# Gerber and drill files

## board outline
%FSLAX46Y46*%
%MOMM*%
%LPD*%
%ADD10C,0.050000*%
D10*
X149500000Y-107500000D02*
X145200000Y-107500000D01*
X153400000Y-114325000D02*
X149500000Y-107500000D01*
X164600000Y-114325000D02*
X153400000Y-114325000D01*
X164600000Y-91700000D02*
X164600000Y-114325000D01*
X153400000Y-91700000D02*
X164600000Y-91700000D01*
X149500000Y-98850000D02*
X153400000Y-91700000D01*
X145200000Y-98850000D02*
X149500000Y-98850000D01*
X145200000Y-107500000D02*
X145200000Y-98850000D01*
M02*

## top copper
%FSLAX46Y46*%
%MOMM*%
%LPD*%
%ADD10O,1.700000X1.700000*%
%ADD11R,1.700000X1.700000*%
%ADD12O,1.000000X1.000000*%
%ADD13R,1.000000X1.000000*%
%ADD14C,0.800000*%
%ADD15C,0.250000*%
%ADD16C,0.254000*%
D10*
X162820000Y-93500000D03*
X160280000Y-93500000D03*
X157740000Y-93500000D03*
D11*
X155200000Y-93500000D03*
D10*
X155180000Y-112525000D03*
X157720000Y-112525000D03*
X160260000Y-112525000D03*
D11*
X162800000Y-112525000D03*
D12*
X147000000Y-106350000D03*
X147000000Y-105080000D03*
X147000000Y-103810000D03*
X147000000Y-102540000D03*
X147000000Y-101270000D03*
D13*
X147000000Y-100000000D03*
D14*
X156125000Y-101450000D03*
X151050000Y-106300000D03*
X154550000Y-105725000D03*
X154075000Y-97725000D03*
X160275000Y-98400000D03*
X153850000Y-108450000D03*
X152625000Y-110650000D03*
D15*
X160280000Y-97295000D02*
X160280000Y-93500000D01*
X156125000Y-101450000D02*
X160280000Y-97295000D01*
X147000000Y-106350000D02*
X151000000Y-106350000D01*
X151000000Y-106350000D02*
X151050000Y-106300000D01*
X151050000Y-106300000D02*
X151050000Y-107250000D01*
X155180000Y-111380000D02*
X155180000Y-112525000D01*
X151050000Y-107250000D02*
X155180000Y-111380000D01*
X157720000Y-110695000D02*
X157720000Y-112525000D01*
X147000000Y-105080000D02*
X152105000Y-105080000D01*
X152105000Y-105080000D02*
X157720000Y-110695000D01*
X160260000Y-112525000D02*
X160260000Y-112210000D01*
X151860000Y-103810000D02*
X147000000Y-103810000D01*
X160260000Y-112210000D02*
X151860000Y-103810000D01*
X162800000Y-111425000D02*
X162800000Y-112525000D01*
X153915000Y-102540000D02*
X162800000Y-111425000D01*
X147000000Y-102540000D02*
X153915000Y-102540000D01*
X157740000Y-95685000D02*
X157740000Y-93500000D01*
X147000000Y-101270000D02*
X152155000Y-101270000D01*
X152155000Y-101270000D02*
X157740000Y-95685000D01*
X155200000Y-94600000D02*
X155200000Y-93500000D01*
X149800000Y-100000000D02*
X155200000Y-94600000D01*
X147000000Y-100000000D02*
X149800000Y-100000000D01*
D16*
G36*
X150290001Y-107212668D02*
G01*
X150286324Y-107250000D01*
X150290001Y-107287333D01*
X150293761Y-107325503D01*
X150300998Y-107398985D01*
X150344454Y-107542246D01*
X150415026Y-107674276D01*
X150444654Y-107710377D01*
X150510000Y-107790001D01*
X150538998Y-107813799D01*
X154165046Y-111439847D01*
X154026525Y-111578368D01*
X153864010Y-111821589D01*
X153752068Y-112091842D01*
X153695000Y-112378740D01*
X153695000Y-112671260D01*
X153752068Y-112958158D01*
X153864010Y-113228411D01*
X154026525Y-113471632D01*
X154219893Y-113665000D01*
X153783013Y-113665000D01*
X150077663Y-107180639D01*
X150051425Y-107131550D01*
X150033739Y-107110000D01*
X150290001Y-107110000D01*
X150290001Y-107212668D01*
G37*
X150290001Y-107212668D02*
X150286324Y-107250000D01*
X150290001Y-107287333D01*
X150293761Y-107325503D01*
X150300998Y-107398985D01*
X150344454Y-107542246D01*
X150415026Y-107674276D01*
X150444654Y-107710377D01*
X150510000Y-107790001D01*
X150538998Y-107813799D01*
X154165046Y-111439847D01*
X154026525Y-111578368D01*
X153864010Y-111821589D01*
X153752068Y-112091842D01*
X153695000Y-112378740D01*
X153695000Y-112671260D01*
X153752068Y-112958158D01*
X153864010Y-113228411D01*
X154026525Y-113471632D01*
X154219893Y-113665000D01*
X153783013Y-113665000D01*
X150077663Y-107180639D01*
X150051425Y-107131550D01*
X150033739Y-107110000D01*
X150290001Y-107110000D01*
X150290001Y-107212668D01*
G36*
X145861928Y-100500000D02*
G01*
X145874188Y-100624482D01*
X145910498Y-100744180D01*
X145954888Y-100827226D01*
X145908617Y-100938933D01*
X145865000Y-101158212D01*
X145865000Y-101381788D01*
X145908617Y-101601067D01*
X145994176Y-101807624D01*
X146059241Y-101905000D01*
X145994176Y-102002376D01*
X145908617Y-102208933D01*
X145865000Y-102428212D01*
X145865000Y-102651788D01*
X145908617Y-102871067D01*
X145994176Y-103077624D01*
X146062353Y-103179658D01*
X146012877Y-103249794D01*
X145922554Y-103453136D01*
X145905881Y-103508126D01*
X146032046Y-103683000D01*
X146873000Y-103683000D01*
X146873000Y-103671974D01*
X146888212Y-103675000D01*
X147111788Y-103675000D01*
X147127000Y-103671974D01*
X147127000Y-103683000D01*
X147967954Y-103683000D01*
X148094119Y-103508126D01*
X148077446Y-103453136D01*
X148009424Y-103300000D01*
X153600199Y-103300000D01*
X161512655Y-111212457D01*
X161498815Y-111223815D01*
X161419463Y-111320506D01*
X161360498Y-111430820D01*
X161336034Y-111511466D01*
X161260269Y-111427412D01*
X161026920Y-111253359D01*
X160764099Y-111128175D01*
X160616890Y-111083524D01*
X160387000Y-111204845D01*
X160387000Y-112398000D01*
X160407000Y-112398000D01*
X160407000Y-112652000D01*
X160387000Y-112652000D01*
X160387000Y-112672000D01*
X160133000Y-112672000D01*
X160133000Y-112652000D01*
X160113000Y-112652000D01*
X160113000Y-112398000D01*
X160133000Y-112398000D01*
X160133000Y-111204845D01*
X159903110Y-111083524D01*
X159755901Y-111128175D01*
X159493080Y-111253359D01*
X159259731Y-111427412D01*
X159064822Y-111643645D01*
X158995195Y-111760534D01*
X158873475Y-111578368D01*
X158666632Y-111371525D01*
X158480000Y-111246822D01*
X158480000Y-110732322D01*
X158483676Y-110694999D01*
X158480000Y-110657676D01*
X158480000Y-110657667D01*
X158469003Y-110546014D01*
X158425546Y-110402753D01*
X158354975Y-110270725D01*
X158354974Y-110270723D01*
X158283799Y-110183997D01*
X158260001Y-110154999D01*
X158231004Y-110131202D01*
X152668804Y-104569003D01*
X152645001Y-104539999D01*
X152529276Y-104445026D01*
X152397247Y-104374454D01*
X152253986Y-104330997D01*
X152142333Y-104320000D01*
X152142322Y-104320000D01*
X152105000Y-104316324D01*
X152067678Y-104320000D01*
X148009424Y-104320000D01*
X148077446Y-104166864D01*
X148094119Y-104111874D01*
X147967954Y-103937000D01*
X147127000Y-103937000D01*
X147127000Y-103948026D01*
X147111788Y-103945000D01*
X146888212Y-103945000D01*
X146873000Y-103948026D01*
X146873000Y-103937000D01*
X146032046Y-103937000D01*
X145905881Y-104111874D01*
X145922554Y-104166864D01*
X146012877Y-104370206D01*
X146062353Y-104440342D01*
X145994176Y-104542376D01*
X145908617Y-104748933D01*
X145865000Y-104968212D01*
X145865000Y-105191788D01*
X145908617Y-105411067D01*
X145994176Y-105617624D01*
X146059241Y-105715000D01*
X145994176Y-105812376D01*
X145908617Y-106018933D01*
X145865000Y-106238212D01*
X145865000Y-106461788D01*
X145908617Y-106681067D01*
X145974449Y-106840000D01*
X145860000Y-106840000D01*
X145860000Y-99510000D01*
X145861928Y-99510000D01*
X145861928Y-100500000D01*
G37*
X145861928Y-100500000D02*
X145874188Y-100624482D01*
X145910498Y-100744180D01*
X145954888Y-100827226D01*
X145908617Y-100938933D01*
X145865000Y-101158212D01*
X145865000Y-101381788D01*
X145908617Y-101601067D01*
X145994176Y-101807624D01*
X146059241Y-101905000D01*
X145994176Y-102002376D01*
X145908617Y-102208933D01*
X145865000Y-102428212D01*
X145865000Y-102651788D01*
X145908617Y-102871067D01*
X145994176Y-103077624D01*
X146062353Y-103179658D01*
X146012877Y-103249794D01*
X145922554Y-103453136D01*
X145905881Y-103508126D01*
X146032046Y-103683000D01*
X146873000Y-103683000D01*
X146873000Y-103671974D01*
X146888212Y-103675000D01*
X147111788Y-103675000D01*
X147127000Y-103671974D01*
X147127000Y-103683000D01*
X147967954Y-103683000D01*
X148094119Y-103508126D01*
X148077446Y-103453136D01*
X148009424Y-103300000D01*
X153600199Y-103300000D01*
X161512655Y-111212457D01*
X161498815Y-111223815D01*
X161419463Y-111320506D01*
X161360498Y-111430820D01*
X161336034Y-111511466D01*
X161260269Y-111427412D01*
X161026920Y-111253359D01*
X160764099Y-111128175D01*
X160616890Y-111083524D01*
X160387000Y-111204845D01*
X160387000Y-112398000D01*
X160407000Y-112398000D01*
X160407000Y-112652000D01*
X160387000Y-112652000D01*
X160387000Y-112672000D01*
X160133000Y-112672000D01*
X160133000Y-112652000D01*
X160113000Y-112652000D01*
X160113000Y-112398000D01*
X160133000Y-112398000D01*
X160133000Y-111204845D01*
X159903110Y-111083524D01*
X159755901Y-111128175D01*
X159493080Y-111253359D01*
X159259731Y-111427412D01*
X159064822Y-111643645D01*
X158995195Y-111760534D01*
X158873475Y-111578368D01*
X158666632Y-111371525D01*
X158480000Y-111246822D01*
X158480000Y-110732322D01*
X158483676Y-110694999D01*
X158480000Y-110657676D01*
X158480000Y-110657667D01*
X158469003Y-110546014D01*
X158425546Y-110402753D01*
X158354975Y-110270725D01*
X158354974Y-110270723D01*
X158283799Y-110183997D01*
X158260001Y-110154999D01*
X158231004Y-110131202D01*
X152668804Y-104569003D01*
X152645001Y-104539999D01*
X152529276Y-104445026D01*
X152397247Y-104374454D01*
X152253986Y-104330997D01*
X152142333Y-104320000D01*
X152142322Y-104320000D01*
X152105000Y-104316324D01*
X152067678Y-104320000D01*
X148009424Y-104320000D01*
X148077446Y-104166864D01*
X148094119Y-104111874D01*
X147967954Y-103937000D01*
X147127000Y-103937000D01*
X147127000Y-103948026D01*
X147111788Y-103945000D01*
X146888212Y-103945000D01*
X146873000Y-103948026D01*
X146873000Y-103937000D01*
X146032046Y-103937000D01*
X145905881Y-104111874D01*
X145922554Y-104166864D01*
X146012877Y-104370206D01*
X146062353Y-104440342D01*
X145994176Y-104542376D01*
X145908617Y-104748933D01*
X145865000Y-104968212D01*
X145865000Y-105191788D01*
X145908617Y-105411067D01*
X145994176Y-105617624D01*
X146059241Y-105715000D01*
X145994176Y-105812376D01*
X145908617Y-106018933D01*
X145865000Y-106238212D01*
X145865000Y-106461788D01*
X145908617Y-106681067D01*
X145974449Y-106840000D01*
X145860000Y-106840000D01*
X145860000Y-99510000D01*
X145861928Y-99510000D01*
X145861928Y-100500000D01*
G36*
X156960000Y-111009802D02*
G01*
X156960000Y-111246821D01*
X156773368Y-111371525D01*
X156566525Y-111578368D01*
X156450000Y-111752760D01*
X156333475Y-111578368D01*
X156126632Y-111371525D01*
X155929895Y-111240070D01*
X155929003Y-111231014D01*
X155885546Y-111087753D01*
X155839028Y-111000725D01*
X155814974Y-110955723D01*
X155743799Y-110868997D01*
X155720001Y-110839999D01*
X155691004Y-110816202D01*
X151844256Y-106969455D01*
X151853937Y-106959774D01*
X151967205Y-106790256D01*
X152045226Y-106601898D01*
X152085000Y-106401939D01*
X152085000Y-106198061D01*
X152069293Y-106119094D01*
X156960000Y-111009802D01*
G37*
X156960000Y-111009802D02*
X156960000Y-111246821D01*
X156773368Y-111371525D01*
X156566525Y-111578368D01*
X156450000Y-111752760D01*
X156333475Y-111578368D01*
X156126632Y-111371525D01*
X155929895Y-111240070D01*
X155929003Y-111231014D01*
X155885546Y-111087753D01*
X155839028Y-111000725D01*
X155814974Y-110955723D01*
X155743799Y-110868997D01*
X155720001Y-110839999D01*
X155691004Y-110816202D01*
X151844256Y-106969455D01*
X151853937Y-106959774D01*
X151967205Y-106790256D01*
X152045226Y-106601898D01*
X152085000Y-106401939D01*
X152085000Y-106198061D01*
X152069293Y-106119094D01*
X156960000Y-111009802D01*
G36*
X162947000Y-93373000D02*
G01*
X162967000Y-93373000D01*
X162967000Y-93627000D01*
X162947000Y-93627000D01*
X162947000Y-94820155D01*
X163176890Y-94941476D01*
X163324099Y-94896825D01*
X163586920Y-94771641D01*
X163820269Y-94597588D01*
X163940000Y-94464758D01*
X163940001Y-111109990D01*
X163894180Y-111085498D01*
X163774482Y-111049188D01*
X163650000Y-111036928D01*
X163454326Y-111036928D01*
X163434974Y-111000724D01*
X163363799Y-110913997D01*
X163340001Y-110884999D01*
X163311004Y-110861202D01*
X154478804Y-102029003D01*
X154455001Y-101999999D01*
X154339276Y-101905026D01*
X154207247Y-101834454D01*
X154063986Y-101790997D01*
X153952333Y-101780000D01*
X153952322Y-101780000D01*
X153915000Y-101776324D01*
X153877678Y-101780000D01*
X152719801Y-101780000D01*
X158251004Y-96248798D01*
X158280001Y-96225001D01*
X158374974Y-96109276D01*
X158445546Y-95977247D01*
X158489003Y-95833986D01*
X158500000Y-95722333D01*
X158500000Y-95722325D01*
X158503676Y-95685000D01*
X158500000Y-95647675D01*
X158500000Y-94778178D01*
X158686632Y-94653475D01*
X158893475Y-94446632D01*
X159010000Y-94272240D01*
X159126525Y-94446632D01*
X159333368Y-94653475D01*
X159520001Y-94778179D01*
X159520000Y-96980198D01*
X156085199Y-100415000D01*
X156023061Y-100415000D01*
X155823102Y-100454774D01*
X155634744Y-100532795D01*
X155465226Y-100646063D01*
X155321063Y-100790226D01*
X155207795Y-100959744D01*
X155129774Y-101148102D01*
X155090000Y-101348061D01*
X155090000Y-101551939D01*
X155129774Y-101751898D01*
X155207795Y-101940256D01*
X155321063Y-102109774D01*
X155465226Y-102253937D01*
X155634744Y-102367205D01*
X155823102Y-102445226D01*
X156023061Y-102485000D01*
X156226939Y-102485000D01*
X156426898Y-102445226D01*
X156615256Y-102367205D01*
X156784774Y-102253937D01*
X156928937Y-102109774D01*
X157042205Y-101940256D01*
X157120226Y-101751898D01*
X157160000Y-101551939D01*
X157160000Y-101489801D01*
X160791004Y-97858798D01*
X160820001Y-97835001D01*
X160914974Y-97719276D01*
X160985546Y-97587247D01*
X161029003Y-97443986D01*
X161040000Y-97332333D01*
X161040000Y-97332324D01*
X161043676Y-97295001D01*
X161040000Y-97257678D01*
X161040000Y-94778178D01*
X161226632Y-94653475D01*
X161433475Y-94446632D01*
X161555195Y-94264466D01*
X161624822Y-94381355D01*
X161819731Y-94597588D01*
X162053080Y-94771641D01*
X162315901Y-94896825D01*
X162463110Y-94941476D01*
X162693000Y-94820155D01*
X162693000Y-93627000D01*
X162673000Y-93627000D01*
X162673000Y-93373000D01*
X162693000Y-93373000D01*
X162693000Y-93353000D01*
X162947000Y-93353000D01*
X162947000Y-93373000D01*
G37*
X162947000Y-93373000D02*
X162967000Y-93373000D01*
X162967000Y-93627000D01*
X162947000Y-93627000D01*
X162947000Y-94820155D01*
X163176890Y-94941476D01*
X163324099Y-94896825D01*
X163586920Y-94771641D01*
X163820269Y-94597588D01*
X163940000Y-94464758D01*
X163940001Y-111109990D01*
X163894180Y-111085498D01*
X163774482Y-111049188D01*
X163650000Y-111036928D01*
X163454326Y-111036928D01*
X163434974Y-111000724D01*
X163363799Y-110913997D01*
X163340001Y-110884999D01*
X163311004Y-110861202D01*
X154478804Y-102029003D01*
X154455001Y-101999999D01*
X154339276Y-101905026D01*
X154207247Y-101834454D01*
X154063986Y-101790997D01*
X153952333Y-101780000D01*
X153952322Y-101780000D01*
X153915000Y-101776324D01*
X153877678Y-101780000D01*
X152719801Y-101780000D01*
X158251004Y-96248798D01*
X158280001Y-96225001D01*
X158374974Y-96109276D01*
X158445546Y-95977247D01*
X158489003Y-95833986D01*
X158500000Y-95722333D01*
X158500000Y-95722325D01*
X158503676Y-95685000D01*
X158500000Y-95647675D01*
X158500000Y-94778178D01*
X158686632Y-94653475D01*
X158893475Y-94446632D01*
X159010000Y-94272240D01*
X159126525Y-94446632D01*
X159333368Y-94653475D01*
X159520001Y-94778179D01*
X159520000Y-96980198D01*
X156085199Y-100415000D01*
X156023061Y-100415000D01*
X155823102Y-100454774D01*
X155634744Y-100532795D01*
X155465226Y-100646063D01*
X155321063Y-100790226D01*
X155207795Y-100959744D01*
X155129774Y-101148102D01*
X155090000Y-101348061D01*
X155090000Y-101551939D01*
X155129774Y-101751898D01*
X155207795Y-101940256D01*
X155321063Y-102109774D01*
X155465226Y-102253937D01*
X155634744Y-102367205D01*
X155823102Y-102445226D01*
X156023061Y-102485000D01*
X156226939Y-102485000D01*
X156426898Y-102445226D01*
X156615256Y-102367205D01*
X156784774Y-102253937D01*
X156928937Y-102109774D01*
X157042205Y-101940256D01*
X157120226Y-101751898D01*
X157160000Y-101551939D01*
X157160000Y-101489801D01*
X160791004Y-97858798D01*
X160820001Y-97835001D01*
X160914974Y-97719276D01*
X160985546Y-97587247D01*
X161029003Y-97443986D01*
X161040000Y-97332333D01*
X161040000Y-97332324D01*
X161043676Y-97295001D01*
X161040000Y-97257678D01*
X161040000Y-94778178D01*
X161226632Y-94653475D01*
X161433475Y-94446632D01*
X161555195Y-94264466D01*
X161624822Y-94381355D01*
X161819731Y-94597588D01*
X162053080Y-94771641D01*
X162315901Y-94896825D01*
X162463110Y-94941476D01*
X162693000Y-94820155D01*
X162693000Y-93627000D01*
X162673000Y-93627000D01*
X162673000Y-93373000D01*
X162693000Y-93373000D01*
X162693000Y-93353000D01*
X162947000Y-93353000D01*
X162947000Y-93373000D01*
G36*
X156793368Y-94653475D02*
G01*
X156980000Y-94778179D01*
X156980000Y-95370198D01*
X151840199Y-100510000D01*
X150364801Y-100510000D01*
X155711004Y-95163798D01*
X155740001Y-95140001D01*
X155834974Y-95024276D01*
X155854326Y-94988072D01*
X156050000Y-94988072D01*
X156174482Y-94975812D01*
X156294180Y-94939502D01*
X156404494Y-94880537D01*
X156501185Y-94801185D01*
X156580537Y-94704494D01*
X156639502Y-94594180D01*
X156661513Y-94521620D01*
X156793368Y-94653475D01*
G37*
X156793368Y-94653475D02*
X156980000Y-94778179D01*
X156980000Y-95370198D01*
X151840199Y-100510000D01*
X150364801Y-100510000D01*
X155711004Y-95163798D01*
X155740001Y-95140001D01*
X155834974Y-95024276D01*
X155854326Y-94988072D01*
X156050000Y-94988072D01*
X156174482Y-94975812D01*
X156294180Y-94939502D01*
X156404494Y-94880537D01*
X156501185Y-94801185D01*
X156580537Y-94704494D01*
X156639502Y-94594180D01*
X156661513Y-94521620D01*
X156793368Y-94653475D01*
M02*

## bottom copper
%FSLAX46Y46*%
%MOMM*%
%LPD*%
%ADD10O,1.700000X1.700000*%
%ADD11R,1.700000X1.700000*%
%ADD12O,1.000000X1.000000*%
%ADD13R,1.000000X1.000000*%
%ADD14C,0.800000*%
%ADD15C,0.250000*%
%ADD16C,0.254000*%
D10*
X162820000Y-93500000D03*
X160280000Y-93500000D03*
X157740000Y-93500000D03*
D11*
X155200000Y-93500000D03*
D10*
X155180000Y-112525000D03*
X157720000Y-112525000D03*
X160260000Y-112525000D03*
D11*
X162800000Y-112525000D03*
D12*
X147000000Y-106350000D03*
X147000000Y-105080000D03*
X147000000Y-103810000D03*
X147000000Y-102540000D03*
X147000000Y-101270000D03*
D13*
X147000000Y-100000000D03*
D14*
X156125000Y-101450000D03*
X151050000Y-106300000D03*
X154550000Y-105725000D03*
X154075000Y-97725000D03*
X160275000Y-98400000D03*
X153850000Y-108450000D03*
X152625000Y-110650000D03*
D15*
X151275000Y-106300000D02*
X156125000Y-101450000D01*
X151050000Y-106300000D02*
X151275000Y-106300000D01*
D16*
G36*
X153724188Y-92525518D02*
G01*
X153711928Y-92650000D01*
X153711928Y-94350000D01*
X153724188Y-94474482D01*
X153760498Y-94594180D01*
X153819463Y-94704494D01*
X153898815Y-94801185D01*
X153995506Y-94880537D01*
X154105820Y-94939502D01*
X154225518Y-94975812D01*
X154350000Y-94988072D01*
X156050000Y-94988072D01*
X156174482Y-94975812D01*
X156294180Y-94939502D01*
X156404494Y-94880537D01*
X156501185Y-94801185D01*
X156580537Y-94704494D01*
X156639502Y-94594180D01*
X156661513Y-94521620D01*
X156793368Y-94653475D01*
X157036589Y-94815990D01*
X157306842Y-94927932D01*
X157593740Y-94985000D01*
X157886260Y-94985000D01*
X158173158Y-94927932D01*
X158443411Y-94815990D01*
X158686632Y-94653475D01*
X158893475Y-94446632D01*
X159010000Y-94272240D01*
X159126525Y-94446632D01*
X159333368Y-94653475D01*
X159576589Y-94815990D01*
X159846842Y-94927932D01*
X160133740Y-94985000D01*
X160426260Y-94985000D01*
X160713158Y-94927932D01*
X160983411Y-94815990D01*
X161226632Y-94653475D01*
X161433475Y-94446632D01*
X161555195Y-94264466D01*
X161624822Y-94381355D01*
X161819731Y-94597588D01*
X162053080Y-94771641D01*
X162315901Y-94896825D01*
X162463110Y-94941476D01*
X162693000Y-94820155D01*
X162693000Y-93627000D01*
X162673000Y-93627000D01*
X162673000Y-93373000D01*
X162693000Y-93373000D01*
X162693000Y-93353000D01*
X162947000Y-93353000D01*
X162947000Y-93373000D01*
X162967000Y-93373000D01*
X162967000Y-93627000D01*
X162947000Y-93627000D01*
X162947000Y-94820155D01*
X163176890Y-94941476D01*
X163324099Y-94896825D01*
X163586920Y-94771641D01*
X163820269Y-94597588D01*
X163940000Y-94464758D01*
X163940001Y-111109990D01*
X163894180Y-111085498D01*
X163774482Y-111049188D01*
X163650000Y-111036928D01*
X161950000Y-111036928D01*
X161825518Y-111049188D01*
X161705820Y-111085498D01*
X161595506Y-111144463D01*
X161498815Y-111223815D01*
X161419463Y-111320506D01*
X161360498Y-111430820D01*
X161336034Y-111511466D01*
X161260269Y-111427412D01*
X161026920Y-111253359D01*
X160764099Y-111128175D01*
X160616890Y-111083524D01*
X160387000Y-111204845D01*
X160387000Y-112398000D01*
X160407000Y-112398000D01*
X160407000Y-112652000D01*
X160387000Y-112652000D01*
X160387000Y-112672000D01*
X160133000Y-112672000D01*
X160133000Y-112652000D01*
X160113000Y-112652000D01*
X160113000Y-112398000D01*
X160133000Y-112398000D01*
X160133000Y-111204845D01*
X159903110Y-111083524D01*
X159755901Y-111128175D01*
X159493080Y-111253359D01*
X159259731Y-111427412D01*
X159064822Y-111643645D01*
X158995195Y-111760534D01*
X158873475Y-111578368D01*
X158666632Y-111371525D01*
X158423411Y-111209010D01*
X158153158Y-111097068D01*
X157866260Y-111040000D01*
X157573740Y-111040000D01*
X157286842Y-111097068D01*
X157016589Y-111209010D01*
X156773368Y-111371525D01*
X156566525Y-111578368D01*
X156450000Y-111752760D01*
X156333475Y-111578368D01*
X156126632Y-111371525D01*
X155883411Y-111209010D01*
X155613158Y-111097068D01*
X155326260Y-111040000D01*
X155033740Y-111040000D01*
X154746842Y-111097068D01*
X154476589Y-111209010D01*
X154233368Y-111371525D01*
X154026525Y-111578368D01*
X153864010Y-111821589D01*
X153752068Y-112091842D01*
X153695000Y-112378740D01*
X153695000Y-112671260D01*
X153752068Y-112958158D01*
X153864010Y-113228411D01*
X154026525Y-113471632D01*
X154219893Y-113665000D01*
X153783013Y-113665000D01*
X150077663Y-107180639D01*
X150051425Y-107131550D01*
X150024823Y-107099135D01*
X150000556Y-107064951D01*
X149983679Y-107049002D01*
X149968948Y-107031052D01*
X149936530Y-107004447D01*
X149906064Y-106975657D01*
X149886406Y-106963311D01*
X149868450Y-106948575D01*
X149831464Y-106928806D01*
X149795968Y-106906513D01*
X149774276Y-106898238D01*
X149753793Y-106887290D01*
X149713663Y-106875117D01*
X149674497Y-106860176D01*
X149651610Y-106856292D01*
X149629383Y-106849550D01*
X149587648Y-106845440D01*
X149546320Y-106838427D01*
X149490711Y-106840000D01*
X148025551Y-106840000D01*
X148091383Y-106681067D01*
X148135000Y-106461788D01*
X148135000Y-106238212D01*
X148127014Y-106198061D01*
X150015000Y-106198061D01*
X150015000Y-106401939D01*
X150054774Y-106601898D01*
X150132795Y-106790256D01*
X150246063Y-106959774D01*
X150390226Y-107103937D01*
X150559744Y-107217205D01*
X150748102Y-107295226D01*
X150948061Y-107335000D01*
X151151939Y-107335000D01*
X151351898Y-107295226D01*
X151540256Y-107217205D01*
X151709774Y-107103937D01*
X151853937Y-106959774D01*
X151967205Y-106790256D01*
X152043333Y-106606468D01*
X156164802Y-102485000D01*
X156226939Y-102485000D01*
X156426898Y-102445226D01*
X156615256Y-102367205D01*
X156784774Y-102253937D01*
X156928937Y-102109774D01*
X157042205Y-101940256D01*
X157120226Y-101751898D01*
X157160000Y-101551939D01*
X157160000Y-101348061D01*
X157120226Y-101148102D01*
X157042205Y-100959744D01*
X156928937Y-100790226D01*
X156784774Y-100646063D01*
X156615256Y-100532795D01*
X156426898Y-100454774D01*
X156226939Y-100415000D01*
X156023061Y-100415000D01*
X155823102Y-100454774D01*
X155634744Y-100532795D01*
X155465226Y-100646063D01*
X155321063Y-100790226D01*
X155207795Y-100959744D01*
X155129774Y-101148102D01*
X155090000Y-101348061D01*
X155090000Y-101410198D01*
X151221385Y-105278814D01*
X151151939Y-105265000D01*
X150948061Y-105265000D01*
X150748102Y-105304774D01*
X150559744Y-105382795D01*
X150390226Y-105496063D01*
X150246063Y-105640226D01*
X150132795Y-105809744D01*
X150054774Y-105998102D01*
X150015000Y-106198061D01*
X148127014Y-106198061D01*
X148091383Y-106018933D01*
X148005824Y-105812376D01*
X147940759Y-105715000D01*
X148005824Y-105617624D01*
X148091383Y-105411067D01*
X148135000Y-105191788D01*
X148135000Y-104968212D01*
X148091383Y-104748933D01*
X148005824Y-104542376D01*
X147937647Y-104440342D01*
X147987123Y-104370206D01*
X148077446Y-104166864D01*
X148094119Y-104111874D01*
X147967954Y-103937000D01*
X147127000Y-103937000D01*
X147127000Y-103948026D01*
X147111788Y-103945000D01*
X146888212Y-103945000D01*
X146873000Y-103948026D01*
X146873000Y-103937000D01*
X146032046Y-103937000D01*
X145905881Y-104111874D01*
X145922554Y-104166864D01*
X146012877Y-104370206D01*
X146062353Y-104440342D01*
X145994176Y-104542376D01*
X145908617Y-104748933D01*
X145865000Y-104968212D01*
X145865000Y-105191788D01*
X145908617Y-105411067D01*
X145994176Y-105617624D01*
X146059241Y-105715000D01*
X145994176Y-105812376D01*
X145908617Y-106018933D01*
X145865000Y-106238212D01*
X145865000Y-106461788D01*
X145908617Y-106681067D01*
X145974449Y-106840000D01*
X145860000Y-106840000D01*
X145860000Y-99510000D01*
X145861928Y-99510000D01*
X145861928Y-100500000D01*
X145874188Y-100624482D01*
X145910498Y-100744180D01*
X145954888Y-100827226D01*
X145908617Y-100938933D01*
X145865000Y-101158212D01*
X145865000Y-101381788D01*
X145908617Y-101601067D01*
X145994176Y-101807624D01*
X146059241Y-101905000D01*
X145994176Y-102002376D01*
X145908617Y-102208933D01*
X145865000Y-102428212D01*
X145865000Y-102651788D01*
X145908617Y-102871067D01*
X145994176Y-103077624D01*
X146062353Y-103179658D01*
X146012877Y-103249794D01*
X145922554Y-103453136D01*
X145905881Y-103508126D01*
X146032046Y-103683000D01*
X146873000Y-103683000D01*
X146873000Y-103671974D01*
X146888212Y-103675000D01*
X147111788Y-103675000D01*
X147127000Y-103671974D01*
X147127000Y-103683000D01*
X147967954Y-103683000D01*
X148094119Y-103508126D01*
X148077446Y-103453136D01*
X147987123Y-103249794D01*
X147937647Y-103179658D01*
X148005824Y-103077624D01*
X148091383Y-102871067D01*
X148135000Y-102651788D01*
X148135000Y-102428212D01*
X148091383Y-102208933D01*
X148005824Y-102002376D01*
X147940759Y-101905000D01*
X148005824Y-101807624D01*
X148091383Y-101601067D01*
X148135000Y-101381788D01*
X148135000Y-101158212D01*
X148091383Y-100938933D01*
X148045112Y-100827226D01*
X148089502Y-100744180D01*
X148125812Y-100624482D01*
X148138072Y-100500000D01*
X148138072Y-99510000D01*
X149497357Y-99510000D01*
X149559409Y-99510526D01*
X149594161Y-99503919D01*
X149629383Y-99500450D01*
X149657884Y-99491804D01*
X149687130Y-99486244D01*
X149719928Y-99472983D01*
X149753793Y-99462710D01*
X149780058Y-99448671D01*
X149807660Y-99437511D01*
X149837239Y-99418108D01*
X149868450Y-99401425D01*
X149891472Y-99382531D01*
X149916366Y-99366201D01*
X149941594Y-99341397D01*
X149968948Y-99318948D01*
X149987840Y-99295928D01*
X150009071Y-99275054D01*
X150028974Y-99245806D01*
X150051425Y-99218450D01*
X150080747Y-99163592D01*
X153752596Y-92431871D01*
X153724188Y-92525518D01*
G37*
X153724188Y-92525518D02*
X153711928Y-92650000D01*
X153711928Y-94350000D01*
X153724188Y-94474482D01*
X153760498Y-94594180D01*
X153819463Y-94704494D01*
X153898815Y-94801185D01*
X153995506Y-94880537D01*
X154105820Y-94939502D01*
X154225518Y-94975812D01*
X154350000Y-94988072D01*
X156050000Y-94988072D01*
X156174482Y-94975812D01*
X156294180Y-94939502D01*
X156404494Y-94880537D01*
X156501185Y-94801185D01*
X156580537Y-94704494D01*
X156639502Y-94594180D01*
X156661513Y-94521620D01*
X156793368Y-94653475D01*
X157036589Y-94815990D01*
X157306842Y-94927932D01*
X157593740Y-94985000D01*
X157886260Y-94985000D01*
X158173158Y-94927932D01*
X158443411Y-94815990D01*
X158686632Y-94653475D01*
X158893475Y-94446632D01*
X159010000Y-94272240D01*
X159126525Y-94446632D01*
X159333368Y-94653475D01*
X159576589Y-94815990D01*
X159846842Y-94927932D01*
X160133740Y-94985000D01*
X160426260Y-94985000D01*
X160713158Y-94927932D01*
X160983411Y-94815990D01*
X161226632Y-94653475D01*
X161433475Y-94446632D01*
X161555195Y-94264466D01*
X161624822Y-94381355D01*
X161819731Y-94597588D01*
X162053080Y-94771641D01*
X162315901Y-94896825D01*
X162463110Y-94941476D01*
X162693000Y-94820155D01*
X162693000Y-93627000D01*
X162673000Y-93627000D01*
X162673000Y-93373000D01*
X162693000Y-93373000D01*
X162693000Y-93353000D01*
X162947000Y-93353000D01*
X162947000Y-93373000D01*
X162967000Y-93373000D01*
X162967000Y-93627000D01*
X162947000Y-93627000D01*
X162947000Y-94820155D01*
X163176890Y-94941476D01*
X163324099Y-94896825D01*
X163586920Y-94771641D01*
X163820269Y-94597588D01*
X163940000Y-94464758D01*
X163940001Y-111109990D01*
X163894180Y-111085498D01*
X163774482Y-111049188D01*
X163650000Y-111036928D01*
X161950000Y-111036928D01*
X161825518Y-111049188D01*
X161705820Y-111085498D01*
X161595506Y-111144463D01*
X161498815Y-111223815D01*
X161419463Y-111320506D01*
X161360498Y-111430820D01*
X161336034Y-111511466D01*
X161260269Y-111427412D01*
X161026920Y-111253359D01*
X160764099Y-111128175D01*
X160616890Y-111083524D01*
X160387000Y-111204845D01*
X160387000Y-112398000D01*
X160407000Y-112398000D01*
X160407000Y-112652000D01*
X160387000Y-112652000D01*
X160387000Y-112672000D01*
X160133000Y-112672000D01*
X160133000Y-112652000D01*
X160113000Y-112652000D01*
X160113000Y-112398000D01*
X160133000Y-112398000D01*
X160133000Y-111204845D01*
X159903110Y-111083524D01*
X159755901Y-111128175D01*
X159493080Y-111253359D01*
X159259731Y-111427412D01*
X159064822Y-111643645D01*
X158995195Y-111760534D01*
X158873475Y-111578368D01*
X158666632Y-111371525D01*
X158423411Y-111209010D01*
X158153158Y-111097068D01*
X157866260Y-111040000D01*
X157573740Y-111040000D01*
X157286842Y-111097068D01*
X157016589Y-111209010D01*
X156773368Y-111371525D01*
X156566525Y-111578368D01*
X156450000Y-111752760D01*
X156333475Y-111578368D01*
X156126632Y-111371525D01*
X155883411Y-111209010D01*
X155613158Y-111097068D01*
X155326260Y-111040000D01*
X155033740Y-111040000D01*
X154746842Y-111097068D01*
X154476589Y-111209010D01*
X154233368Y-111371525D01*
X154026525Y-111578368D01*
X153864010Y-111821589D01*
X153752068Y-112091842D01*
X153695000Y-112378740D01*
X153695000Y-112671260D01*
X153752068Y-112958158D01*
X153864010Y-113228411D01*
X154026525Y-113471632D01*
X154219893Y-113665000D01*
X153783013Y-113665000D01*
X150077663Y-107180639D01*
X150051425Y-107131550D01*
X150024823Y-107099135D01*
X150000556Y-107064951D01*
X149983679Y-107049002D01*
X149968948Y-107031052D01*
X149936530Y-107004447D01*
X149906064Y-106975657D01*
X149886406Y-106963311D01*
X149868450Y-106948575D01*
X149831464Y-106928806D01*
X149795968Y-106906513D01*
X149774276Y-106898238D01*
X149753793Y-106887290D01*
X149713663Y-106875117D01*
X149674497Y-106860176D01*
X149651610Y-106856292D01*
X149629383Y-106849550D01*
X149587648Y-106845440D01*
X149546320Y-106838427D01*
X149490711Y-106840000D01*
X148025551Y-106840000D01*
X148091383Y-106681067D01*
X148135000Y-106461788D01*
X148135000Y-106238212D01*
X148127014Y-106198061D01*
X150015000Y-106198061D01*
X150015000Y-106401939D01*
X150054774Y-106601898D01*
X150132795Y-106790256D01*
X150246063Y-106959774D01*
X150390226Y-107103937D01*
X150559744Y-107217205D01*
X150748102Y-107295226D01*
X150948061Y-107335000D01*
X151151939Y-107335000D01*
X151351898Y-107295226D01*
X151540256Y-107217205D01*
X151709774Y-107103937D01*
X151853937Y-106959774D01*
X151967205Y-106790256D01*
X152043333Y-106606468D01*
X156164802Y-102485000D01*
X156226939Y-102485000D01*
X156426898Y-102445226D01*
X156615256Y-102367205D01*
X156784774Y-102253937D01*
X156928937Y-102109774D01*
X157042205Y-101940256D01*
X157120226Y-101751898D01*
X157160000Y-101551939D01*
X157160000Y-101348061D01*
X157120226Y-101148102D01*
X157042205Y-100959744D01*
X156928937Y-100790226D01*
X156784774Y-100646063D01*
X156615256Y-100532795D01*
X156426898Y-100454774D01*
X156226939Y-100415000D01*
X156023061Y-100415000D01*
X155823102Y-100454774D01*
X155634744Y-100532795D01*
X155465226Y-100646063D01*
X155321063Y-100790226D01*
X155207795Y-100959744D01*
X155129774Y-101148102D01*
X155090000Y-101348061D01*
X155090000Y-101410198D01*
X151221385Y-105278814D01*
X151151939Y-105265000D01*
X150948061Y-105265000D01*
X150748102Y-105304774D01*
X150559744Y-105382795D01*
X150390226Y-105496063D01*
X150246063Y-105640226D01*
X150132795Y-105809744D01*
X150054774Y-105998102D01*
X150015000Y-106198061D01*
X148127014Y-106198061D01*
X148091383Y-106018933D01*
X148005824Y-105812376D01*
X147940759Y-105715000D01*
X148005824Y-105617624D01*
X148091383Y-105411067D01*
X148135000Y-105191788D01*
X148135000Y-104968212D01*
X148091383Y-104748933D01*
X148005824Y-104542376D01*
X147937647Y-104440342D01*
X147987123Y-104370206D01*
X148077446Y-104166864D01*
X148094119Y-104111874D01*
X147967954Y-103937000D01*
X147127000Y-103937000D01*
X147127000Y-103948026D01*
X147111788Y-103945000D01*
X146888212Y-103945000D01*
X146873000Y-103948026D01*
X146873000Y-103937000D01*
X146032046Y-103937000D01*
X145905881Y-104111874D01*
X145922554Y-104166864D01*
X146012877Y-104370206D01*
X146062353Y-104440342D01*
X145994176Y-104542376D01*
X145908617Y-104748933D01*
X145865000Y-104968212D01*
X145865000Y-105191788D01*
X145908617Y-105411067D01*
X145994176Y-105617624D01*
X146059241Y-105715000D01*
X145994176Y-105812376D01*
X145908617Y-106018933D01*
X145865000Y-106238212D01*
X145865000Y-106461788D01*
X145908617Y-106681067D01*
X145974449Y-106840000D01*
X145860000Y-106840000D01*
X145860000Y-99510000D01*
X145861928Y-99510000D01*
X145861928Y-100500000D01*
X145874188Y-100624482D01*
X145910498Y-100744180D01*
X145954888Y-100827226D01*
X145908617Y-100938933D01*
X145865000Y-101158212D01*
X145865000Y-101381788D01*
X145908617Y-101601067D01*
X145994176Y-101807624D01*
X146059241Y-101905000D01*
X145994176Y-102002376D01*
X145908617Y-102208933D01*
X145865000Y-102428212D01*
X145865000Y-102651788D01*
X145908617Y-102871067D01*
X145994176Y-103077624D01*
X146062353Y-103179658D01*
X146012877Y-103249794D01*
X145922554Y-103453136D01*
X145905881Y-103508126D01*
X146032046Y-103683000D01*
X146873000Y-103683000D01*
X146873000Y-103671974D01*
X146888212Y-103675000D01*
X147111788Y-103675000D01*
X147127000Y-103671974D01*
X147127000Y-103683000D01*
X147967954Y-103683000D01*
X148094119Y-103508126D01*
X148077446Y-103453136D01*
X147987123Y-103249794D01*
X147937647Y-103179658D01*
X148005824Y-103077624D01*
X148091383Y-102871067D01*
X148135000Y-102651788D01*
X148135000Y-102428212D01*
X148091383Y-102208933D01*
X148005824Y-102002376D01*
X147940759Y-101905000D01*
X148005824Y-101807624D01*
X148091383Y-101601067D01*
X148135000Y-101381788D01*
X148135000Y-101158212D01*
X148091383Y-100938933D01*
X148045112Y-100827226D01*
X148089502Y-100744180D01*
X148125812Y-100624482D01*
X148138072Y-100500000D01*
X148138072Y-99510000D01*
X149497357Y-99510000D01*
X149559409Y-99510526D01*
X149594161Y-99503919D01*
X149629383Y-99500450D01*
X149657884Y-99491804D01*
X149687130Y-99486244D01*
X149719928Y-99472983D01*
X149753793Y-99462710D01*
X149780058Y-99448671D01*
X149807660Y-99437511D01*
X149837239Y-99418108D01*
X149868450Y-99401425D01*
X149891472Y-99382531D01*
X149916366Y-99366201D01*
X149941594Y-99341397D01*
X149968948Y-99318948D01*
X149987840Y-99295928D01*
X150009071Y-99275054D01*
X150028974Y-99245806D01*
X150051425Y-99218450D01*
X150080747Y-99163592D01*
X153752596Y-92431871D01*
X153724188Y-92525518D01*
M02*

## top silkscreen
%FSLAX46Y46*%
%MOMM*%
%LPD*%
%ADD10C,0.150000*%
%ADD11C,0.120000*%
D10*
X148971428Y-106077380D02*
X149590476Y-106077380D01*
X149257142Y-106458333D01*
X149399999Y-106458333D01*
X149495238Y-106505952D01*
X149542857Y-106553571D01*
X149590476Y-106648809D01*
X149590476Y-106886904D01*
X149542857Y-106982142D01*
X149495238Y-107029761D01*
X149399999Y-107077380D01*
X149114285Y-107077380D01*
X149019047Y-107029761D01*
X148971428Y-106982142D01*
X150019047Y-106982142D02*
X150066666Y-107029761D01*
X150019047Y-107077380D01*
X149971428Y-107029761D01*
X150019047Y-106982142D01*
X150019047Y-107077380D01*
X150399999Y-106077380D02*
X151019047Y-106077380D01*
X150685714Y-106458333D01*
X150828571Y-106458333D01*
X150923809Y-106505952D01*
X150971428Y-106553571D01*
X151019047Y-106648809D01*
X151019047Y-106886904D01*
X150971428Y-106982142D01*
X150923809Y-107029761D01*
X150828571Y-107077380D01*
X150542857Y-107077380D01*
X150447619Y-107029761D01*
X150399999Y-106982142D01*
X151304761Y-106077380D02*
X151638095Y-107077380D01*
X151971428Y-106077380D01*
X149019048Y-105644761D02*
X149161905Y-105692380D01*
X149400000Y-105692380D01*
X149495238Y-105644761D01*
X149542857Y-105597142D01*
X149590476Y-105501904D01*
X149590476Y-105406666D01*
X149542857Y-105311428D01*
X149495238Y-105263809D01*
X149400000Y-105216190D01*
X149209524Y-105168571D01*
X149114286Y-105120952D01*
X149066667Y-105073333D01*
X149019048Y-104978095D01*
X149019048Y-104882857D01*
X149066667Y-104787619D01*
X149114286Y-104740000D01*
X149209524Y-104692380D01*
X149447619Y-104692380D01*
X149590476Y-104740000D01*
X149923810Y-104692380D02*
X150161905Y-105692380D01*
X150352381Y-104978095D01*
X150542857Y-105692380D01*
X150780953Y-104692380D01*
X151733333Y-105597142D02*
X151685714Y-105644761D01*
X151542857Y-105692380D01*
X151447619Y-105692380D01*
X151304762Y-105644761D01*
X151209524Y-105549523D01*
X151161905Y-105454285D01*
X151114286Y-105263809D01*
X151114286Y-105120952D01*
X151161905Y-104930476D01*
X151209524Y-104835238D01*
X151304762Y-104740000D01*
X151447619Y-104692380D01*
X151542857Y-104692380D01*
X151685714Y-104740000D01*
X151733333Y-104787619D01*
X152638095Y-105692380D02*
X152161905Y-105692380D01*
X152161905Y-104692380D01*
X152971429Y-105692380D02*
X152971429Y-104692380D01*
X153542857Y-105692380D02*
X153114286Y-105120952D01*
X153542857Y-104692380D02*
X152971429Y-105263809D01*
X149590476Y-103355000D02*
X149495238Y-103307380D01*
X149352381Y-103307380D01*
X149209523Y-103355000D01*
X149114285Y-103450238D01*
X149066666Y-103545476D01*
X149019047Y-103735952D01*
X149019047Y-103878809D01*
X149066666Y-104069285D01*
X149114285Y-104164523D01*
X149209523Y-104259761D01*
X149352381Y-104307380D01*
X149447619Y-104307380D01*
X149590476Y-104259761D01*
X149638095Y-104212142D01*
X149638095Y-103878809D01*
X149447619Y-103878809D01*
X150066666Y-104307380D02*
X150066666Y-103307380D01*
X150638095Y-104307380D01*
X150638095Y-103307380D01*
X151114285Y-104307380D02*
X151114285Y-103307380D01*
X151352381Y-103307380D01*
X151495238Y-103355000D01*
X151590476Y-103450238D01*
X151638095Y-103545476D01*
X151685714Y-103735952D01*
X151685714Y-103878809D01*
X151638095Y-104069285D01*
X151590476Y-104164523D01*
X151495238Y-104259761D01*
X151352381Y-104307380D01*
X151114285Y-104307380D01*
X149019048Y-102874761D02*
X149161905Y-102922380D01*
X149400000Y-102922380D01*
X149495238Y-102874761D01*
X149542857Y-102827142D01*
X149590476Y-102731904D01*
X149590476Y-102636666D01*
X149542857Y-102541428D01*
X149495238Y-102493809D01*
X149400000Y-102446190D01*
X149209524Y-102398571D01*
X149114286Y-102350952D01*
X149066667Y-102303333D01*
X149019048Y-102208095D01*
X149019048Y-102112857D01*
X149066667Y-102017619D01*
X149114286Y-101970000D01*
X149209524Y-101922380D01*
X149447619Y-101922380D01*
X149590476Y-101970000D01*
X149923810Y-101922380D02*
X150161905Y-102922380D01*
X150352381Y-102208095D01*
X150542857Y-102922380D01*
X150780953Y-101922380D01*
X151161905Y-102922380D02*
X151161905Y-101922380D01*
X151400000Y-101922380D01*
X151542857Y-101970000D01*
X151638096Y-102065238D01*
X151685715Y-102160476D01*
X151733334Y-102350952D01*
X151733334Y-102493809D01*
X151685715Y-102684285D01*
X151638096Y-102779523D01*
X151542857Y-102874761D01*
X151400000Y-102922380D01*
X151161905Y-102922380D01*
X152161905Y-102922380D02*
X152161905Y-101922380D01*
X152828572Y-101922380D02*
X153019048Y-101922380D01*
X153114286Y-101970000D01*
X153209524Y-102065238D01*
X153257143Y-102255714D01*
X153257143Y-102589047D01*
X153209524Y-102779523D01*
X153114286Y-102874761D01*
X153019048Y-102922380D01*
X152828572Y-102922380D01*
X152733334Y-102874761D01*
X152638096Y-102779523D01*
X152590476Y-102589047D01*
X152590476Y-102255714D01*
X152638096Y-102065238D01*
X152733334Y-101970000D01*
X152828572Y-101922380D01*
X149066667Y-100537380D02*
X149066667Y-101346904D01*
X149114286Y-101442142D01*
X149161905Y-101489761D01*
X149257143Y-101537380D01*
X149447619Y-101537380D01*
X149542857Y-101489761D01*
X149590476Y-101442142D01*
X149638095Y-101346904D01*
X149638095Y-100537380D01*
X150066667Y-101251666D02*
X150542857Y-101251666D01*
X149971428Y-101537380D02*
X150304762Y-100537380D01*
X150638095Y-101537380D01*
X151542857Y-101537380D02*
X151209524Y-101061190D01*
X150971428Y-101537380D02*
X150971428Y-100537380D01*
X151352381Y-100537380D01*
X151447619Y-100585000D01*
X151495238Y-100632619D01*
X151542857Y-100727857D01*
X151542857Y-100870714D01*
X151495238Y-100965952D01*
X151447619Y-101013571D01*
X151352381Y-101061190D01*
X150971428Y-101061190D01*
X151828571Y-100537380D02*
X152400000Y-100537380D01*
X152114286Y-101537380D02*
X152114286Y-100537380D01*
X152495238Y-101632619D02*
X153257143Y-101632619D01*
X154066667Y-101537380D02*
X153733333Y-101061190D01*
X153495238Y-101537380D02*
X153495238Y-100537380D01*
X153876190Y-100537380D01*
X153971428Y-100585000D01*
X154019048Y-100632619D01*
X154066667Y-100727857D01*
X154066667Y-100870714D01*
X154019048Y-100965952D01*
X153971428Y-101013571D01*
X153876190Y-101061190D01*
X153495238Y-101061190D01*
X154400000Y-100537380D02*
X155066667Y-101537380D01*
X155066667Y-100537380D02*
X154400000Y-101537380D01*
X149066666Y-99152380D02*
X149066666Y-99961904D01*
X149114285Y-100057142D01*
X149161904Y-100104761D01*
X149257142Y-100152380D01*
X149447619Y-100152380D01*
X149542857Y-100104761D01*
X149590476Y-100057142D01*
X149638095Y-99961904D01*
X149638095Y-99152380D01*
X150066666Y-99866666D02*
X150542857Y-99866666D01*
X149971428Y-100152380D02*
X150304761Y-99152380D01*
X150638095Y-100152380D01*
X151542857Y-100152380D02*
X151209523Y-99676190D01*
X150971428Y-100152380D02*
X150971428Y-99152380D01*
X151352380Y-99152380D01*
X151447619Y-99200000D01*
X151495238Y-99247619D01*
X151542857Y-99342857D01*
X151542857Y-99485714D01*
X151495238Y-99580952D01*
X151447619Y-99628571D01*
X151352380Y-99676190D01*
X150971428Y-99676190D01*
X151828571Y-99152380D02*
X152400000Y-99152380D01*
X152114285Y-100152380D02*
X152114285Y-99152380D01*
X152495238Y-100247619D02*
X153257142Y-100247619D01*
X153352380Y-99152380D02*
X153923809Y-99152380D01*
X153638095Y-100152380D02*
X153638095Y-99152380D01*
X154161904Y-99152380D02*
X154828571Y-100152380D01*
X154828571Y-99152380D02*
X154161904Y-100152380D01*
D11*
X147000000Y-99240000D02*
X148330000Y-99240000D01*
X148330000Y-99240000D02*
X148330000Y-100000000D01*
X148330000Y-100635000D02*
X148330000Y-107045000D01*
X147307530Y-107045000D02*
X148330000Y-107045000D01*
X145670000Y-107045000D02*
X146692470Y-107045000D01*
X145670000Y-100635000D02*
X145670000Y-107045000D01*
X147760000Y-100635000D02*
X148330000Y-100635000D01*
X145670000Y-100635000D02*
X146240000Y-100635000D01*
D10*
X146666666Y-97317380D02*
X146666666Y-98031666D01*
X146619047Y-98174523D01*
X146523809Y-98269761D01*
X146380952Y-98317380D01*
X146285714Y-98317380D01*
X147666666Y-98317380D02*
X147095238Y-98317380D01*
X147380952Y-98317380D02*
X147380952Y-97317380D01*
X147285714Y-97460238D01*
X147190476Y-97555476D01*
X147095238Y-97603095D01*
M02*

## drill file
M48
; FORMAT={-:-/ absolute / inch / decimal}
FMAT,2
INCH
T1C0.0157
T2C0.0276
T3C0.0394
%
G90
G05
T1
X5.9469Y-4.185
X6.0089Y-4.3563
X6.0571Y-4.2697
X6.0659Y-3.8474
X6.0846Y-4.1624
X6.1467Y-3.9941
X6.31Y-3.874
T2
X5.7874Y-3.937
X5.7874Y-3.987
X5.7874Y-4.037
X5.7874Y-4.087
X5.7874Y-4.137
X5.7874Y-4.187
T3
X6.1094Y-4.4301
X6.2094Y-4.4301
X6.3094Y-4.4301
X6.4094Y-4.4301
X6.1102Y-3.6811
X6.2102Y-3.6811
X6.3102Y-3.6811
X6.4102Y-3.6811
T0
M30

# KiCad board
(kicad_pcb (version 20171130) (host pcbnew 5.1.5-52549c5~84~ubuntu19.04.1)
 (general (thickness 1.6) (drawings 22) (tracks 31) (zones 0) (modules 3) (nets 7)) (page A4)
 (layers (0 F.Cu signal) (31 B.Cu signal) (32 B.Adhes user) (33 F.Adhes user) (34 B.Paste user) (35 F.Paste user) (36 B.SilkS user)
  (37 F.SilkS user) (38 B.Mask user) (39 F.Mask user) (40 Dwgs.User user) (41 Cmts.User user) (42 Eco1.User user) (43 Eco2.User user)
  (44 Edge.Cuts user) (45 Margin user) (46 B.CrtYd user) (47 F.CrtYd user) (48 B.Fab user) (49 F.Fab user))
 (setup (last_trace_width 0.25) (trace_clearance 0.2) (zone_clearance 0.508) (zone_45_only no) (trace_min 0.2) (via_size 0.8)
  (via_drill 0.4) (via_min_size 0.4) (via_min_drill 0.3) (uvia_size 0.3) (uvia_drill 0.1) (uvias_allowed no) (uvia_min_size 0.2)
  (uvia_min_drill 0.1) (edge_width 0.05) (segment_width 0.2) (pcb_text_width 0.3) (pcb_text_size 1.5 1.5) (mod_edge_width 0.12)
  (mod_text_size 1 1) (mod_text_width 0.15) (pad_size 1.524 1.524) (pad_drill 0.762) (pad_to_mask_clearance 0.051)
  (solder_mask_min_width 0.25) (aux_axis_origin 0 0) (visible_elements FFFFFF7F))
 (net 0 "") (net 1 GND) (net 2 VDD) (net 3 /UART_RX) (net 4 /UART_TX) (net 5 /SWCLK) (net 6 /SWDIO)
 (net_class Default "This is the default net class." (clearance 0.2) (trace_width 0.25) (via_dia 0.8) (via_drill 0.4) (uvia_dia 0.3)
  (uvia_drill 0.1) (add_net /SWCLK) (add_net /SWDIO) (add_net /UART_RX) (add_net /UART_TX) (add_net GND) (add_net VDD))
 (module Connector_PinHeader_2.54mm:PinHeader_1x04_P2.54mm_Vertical (layer B.Cu) (at 155.2 93.5 270)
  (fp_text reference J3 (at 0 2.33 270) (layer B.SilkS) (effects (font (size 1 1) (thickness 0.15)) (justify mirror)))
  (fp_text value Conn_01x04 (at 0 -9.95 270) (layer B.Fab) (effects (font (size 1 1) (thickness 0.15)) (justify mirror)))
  (pad 4 thru_hole oval (at 0 -7.62 270) (size 1.7 1.7) (drill 1) (layers *.Cu *.Mask) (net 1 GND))
  (pad 3 thru_hole oval (at 0 -5.08 270) (size 1.7 1.7) (drill 1) (layers *.Cu *.Mask) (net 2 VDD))
  (pad 2 thru_hole oval (at 0 -2.54 270) (size 1.7 1.7) (drill 1) (layers *.Cu *.Mask) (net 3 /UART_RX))
  (pad 1 thru_hole rect (at 0 0 270) (size 1.7 1.7) (drill 1) (layers *.Cu *.Mask) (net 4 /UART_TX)))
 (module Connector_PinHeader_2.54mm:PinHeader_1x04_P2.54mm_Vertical (layer B.Cu) (at 162.8 112.525 90)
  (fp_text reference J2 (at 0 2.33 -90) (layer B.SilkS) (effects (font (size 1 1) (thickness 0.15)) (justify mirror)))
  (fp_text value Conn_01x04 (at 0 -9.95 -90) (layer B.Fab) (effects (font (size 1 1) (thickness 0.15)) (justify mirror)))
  (pad 4 thru_hole oval (at 0 -7.62 90) (size 1.7 1.7) (drill 1) (layers *.Cu *.Mask) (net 2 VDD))
  (pad 3 thru_hole oval (at 0 -5.08 90) (size 1.7 1.7) (drill 1) (layers *.Cu *.Mask) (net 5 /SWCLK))
  (pad 2 thru_hole oval (at 0 -2.54 90) (size 1.7 1.7) (drill 1) (layers *.Cu *.Mask) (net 1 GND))
  (pad 1 thru_hole rect (at 0 0 90) (size 1.7 1.7) (drill 1) (layers *.Cu *.Mask) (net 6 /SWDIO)))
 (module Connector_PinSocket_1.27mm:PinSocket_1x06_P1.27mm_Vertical (layer F.Cu) (at 147 100)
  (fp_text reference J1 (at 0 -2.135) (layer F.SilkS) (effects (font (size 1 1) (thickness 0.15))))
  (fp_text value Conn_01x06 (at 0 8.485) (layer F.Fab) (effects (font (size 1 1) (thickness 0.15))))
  (fp_line (start 0 -0.76) (end 1.33 -0.76) (layer F.SilkS) (width 0.12))
  (fp_line (start 1.33 -0.76) (end 1.33 0) (layer F.SilkS) (width 0.12))
  (fp_line (start 1.33 0.635) (end 1.33 7.045) (layer F.SilkS) (width 0.12))
  (fp_line (start 0.30753 7.045) (end 1.33 7.045) (layer F.SilkS) (width 0.12))
  (fp_line (start -1.33 7.045) (end -0.30753 7.045) (layer F.SilkS) (width 0.12))
  (fp_line (start -1.33 0.635) (end -1.33 7.045) (layer F.SilkS) (width 0.12))
  (fp_line (start 0.76 0.635) (end 1.33 0.635) (layer F.SilkS) (width 0.12))
  (fp_line (start -1.33 0.635) (end -0.76 0.635) (layer F.SilkS) (width 0.12))
  (pad 6 thru_hole oval (at 0 6.35) (size 1 1) (drill 0.7) (layers *.Cu *.Mask) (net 2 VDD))
  (pad 5 thru_hole oval (at 0 5.08) (size 1 1) (drill 0.7) (layers *.Cu *.Mask) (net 5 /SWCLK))
  (pad 4 thru_hole oval (at 0 3.81) (size 1 1) (drill 0.7) (layers *.Cu *.Mask) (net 1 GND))
  (pad 3 thru_hole oval (at 0 2.54) (size 1 1) (drill 0.7) (layers *.Cu *.Mask) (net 6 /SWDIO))
  (pad 2 thru_hole oval (at 0 1.27) (size 1 1) (drill 0.7) (layers *.Cu *.Mask) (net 3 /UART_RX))
  (pad 1 thru_hole rect (at 0 0) (size 1 1) (drill 0.7) (layers *.Cu *.Mask) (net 4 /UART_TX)))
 (gr_line (start 149.5 107.5) (end 145.2 107.5) (layer Edge.Cuts) (width 0.05))
 (gr_line (start 153.4 114.325) (end 149.5 107.5) (layer Edge.Cuts) (width 0.05))
 (gr_line (start 164.6 114.325) (end 153.4 114.325) (layer Edge.Cuts) (width 0.05))
 (gr_line (start 164.6 91.7) (end 164.6 114.325) (layer Edge.Cuts) (width 0.05))
 (gr_line (start 153.4 91.7) (end 164.6 91.7) (layer Edge.Cuts) (width 0.05))
 (gr_line (start 149.5 98.85) (end 153.4 91.7) (layer Edge.Cuts) (width 0.05))
 (gr_line (start 145.2 98.85) (end 149.5 98.85) (layer Edge.Cuts) (width 0.05))
 (gr_line (start 145.2 107.5) (end 145.2 98.85) (layer Edge.Cuts) (width 0.05))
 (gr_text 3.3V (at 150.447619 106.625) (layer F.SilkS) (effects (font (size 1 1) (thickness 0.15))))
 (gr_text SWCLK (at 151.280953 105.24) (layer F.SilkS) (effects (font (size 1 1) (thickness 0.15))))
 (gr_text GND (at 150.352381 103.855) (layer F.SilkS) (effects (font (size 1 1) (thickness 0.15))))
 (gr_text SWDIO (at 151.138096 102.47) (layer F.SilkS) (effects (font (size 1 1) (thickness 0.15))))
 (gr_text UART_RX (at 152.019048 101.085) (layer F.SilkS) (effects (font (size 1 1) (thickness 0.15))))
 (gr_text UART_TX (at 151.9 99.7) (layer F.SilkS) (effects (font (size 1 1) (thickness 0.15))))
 (via (at 156.125 101.45) (size 0.8) (drill 0.4) (layers F.Cu B.Cu) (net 2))
 (segment (start 160.28 97.295) (end 160.28 93.5) (width 0.25) (layer F.Cu) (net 2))
 (segment (start 156.125 101.45) (end 160.28 97.295) (width 0.25) (layer F.Cu) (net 2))
 (segment (start 147 106.35) (end 151 106.35) (width 0.25) (layer F.Cu) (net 2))
 (via (at 151.05 106.3) (size 0.8) (drill 0.4) (layers F.Cu B.Cu) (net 2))
 (segment (start 151 106.35) (end 151.05 106.3) (width 0.25) (layer F.Cu) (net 2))
 (segment (start 151.275 106.3) (end 156.125 101.45) (width 0.25) (layer B.Cu) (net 2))
 (segment (start 151.05 106.3) (end 151.275 106.3) (width 0.25) (layer B.Cu) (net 2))
 (segment (start 151.05 106.3) (end 151.05 107.25) (width 0.25) (layer F.Cu) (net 2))
 (segment (start 155.18 111.38) (end 155.18 112.525) (width 0.25) (layer F.Cu) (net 2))
 (segment (start 151.05 107.25) (end 155.18 111.38) (width 0.25) (layer F.Cu) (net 2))
 (segment (start 157.72 110.695) (end 157.72 112.525) (width 0.25) (layer F.Cu) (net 5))
 (segment (start 147 105.08) (end 152.105 105.08) (width 0.25) (layer F.Cu) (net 5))
 (segment (start 152.105 105.08) (end 157.72 110.695) (width 0.25) (layer F.Cu) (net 5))
 (segment (start 160.26 112.525) (end 160.26 112.21) (width 0.25) (layer F.Cu) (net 1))
 (segment (start 151.86 103.81) (end 147 103.81) (width 0.25) (layer F.Cu) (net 1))
 (segment (start 160.26 112.21) (end 151.86 103.81) (width 0.25) (layer F.Cu) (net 1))
 (via (at 154.55 105.725) (size 0.8) (drill 0.4) (layers F.Cu B.Cu) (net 1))
 (via (at 154.075 97.725) (size 0.8) (drill 0.4) (layers F.Cu B.Cu) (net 1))
 (via (at 160.275 98.4) (size 0.8) (drill 0.4) (layers F.Cu B.Cu) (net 1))
 (via (at 153.85 108.45) (size 0.8) (drill 0.4) (layers F.Cu B.Cu) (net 1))
 (via (at 152.625 110.65) (size 0.8) (drill 0.4) (layers F.Cu B.Cu) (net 1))
 (segment (start 162.8 111.425) (end 162.8 112.525) (width 0.25) (layer F.Cu) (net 6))
 (segment (start 153.915 102.54) (end 162.8 111.425) (width 0.25) (layer F.Cu) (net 6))
 (segment (start 147 102.54) (end 153.915 102.54) (width 0.25) (layer F.Cu) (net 6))
 (segment (start 157.74 95.685) (end 157.74 93.5) (width 0.25) (layer F.Cu) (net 3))
 (segment (start 147 101.27) (end 152.155 101.27) (width 0.25) (layer F.Cu) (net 3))
 (segment (start 152.155 101.27) (end 157.74 95.685) (width 0.25) (layer F.Cu) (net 3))
 (segment (start 155.2 94.6) (end 155.2 93.5) (width 0.25) (layer F.Cu) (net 4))
 (segment (start 149.8 100) (end 155.2 94.6) (width 0.25) (layer F.Cu) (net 4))
 (segment (start 147 100) (end 149.8 100) (width 0.25) (layer F.Cu) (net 4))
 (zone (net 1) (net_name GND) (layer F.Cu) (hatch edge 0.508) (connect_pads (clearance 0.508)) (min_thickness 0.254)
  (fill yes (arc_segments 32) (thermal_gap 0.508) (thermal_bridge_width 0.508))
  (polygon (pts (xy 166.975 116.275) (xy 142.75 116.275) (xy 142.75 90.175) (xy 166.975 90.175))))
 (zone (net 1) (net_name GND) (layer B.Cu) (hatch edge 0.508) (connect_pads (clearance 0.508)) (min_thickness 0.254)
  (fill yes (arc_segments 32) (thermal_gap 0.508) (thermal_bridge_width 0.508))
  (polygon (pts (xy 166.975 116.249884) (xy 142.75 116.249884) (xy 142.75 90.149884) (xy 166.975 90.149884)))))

